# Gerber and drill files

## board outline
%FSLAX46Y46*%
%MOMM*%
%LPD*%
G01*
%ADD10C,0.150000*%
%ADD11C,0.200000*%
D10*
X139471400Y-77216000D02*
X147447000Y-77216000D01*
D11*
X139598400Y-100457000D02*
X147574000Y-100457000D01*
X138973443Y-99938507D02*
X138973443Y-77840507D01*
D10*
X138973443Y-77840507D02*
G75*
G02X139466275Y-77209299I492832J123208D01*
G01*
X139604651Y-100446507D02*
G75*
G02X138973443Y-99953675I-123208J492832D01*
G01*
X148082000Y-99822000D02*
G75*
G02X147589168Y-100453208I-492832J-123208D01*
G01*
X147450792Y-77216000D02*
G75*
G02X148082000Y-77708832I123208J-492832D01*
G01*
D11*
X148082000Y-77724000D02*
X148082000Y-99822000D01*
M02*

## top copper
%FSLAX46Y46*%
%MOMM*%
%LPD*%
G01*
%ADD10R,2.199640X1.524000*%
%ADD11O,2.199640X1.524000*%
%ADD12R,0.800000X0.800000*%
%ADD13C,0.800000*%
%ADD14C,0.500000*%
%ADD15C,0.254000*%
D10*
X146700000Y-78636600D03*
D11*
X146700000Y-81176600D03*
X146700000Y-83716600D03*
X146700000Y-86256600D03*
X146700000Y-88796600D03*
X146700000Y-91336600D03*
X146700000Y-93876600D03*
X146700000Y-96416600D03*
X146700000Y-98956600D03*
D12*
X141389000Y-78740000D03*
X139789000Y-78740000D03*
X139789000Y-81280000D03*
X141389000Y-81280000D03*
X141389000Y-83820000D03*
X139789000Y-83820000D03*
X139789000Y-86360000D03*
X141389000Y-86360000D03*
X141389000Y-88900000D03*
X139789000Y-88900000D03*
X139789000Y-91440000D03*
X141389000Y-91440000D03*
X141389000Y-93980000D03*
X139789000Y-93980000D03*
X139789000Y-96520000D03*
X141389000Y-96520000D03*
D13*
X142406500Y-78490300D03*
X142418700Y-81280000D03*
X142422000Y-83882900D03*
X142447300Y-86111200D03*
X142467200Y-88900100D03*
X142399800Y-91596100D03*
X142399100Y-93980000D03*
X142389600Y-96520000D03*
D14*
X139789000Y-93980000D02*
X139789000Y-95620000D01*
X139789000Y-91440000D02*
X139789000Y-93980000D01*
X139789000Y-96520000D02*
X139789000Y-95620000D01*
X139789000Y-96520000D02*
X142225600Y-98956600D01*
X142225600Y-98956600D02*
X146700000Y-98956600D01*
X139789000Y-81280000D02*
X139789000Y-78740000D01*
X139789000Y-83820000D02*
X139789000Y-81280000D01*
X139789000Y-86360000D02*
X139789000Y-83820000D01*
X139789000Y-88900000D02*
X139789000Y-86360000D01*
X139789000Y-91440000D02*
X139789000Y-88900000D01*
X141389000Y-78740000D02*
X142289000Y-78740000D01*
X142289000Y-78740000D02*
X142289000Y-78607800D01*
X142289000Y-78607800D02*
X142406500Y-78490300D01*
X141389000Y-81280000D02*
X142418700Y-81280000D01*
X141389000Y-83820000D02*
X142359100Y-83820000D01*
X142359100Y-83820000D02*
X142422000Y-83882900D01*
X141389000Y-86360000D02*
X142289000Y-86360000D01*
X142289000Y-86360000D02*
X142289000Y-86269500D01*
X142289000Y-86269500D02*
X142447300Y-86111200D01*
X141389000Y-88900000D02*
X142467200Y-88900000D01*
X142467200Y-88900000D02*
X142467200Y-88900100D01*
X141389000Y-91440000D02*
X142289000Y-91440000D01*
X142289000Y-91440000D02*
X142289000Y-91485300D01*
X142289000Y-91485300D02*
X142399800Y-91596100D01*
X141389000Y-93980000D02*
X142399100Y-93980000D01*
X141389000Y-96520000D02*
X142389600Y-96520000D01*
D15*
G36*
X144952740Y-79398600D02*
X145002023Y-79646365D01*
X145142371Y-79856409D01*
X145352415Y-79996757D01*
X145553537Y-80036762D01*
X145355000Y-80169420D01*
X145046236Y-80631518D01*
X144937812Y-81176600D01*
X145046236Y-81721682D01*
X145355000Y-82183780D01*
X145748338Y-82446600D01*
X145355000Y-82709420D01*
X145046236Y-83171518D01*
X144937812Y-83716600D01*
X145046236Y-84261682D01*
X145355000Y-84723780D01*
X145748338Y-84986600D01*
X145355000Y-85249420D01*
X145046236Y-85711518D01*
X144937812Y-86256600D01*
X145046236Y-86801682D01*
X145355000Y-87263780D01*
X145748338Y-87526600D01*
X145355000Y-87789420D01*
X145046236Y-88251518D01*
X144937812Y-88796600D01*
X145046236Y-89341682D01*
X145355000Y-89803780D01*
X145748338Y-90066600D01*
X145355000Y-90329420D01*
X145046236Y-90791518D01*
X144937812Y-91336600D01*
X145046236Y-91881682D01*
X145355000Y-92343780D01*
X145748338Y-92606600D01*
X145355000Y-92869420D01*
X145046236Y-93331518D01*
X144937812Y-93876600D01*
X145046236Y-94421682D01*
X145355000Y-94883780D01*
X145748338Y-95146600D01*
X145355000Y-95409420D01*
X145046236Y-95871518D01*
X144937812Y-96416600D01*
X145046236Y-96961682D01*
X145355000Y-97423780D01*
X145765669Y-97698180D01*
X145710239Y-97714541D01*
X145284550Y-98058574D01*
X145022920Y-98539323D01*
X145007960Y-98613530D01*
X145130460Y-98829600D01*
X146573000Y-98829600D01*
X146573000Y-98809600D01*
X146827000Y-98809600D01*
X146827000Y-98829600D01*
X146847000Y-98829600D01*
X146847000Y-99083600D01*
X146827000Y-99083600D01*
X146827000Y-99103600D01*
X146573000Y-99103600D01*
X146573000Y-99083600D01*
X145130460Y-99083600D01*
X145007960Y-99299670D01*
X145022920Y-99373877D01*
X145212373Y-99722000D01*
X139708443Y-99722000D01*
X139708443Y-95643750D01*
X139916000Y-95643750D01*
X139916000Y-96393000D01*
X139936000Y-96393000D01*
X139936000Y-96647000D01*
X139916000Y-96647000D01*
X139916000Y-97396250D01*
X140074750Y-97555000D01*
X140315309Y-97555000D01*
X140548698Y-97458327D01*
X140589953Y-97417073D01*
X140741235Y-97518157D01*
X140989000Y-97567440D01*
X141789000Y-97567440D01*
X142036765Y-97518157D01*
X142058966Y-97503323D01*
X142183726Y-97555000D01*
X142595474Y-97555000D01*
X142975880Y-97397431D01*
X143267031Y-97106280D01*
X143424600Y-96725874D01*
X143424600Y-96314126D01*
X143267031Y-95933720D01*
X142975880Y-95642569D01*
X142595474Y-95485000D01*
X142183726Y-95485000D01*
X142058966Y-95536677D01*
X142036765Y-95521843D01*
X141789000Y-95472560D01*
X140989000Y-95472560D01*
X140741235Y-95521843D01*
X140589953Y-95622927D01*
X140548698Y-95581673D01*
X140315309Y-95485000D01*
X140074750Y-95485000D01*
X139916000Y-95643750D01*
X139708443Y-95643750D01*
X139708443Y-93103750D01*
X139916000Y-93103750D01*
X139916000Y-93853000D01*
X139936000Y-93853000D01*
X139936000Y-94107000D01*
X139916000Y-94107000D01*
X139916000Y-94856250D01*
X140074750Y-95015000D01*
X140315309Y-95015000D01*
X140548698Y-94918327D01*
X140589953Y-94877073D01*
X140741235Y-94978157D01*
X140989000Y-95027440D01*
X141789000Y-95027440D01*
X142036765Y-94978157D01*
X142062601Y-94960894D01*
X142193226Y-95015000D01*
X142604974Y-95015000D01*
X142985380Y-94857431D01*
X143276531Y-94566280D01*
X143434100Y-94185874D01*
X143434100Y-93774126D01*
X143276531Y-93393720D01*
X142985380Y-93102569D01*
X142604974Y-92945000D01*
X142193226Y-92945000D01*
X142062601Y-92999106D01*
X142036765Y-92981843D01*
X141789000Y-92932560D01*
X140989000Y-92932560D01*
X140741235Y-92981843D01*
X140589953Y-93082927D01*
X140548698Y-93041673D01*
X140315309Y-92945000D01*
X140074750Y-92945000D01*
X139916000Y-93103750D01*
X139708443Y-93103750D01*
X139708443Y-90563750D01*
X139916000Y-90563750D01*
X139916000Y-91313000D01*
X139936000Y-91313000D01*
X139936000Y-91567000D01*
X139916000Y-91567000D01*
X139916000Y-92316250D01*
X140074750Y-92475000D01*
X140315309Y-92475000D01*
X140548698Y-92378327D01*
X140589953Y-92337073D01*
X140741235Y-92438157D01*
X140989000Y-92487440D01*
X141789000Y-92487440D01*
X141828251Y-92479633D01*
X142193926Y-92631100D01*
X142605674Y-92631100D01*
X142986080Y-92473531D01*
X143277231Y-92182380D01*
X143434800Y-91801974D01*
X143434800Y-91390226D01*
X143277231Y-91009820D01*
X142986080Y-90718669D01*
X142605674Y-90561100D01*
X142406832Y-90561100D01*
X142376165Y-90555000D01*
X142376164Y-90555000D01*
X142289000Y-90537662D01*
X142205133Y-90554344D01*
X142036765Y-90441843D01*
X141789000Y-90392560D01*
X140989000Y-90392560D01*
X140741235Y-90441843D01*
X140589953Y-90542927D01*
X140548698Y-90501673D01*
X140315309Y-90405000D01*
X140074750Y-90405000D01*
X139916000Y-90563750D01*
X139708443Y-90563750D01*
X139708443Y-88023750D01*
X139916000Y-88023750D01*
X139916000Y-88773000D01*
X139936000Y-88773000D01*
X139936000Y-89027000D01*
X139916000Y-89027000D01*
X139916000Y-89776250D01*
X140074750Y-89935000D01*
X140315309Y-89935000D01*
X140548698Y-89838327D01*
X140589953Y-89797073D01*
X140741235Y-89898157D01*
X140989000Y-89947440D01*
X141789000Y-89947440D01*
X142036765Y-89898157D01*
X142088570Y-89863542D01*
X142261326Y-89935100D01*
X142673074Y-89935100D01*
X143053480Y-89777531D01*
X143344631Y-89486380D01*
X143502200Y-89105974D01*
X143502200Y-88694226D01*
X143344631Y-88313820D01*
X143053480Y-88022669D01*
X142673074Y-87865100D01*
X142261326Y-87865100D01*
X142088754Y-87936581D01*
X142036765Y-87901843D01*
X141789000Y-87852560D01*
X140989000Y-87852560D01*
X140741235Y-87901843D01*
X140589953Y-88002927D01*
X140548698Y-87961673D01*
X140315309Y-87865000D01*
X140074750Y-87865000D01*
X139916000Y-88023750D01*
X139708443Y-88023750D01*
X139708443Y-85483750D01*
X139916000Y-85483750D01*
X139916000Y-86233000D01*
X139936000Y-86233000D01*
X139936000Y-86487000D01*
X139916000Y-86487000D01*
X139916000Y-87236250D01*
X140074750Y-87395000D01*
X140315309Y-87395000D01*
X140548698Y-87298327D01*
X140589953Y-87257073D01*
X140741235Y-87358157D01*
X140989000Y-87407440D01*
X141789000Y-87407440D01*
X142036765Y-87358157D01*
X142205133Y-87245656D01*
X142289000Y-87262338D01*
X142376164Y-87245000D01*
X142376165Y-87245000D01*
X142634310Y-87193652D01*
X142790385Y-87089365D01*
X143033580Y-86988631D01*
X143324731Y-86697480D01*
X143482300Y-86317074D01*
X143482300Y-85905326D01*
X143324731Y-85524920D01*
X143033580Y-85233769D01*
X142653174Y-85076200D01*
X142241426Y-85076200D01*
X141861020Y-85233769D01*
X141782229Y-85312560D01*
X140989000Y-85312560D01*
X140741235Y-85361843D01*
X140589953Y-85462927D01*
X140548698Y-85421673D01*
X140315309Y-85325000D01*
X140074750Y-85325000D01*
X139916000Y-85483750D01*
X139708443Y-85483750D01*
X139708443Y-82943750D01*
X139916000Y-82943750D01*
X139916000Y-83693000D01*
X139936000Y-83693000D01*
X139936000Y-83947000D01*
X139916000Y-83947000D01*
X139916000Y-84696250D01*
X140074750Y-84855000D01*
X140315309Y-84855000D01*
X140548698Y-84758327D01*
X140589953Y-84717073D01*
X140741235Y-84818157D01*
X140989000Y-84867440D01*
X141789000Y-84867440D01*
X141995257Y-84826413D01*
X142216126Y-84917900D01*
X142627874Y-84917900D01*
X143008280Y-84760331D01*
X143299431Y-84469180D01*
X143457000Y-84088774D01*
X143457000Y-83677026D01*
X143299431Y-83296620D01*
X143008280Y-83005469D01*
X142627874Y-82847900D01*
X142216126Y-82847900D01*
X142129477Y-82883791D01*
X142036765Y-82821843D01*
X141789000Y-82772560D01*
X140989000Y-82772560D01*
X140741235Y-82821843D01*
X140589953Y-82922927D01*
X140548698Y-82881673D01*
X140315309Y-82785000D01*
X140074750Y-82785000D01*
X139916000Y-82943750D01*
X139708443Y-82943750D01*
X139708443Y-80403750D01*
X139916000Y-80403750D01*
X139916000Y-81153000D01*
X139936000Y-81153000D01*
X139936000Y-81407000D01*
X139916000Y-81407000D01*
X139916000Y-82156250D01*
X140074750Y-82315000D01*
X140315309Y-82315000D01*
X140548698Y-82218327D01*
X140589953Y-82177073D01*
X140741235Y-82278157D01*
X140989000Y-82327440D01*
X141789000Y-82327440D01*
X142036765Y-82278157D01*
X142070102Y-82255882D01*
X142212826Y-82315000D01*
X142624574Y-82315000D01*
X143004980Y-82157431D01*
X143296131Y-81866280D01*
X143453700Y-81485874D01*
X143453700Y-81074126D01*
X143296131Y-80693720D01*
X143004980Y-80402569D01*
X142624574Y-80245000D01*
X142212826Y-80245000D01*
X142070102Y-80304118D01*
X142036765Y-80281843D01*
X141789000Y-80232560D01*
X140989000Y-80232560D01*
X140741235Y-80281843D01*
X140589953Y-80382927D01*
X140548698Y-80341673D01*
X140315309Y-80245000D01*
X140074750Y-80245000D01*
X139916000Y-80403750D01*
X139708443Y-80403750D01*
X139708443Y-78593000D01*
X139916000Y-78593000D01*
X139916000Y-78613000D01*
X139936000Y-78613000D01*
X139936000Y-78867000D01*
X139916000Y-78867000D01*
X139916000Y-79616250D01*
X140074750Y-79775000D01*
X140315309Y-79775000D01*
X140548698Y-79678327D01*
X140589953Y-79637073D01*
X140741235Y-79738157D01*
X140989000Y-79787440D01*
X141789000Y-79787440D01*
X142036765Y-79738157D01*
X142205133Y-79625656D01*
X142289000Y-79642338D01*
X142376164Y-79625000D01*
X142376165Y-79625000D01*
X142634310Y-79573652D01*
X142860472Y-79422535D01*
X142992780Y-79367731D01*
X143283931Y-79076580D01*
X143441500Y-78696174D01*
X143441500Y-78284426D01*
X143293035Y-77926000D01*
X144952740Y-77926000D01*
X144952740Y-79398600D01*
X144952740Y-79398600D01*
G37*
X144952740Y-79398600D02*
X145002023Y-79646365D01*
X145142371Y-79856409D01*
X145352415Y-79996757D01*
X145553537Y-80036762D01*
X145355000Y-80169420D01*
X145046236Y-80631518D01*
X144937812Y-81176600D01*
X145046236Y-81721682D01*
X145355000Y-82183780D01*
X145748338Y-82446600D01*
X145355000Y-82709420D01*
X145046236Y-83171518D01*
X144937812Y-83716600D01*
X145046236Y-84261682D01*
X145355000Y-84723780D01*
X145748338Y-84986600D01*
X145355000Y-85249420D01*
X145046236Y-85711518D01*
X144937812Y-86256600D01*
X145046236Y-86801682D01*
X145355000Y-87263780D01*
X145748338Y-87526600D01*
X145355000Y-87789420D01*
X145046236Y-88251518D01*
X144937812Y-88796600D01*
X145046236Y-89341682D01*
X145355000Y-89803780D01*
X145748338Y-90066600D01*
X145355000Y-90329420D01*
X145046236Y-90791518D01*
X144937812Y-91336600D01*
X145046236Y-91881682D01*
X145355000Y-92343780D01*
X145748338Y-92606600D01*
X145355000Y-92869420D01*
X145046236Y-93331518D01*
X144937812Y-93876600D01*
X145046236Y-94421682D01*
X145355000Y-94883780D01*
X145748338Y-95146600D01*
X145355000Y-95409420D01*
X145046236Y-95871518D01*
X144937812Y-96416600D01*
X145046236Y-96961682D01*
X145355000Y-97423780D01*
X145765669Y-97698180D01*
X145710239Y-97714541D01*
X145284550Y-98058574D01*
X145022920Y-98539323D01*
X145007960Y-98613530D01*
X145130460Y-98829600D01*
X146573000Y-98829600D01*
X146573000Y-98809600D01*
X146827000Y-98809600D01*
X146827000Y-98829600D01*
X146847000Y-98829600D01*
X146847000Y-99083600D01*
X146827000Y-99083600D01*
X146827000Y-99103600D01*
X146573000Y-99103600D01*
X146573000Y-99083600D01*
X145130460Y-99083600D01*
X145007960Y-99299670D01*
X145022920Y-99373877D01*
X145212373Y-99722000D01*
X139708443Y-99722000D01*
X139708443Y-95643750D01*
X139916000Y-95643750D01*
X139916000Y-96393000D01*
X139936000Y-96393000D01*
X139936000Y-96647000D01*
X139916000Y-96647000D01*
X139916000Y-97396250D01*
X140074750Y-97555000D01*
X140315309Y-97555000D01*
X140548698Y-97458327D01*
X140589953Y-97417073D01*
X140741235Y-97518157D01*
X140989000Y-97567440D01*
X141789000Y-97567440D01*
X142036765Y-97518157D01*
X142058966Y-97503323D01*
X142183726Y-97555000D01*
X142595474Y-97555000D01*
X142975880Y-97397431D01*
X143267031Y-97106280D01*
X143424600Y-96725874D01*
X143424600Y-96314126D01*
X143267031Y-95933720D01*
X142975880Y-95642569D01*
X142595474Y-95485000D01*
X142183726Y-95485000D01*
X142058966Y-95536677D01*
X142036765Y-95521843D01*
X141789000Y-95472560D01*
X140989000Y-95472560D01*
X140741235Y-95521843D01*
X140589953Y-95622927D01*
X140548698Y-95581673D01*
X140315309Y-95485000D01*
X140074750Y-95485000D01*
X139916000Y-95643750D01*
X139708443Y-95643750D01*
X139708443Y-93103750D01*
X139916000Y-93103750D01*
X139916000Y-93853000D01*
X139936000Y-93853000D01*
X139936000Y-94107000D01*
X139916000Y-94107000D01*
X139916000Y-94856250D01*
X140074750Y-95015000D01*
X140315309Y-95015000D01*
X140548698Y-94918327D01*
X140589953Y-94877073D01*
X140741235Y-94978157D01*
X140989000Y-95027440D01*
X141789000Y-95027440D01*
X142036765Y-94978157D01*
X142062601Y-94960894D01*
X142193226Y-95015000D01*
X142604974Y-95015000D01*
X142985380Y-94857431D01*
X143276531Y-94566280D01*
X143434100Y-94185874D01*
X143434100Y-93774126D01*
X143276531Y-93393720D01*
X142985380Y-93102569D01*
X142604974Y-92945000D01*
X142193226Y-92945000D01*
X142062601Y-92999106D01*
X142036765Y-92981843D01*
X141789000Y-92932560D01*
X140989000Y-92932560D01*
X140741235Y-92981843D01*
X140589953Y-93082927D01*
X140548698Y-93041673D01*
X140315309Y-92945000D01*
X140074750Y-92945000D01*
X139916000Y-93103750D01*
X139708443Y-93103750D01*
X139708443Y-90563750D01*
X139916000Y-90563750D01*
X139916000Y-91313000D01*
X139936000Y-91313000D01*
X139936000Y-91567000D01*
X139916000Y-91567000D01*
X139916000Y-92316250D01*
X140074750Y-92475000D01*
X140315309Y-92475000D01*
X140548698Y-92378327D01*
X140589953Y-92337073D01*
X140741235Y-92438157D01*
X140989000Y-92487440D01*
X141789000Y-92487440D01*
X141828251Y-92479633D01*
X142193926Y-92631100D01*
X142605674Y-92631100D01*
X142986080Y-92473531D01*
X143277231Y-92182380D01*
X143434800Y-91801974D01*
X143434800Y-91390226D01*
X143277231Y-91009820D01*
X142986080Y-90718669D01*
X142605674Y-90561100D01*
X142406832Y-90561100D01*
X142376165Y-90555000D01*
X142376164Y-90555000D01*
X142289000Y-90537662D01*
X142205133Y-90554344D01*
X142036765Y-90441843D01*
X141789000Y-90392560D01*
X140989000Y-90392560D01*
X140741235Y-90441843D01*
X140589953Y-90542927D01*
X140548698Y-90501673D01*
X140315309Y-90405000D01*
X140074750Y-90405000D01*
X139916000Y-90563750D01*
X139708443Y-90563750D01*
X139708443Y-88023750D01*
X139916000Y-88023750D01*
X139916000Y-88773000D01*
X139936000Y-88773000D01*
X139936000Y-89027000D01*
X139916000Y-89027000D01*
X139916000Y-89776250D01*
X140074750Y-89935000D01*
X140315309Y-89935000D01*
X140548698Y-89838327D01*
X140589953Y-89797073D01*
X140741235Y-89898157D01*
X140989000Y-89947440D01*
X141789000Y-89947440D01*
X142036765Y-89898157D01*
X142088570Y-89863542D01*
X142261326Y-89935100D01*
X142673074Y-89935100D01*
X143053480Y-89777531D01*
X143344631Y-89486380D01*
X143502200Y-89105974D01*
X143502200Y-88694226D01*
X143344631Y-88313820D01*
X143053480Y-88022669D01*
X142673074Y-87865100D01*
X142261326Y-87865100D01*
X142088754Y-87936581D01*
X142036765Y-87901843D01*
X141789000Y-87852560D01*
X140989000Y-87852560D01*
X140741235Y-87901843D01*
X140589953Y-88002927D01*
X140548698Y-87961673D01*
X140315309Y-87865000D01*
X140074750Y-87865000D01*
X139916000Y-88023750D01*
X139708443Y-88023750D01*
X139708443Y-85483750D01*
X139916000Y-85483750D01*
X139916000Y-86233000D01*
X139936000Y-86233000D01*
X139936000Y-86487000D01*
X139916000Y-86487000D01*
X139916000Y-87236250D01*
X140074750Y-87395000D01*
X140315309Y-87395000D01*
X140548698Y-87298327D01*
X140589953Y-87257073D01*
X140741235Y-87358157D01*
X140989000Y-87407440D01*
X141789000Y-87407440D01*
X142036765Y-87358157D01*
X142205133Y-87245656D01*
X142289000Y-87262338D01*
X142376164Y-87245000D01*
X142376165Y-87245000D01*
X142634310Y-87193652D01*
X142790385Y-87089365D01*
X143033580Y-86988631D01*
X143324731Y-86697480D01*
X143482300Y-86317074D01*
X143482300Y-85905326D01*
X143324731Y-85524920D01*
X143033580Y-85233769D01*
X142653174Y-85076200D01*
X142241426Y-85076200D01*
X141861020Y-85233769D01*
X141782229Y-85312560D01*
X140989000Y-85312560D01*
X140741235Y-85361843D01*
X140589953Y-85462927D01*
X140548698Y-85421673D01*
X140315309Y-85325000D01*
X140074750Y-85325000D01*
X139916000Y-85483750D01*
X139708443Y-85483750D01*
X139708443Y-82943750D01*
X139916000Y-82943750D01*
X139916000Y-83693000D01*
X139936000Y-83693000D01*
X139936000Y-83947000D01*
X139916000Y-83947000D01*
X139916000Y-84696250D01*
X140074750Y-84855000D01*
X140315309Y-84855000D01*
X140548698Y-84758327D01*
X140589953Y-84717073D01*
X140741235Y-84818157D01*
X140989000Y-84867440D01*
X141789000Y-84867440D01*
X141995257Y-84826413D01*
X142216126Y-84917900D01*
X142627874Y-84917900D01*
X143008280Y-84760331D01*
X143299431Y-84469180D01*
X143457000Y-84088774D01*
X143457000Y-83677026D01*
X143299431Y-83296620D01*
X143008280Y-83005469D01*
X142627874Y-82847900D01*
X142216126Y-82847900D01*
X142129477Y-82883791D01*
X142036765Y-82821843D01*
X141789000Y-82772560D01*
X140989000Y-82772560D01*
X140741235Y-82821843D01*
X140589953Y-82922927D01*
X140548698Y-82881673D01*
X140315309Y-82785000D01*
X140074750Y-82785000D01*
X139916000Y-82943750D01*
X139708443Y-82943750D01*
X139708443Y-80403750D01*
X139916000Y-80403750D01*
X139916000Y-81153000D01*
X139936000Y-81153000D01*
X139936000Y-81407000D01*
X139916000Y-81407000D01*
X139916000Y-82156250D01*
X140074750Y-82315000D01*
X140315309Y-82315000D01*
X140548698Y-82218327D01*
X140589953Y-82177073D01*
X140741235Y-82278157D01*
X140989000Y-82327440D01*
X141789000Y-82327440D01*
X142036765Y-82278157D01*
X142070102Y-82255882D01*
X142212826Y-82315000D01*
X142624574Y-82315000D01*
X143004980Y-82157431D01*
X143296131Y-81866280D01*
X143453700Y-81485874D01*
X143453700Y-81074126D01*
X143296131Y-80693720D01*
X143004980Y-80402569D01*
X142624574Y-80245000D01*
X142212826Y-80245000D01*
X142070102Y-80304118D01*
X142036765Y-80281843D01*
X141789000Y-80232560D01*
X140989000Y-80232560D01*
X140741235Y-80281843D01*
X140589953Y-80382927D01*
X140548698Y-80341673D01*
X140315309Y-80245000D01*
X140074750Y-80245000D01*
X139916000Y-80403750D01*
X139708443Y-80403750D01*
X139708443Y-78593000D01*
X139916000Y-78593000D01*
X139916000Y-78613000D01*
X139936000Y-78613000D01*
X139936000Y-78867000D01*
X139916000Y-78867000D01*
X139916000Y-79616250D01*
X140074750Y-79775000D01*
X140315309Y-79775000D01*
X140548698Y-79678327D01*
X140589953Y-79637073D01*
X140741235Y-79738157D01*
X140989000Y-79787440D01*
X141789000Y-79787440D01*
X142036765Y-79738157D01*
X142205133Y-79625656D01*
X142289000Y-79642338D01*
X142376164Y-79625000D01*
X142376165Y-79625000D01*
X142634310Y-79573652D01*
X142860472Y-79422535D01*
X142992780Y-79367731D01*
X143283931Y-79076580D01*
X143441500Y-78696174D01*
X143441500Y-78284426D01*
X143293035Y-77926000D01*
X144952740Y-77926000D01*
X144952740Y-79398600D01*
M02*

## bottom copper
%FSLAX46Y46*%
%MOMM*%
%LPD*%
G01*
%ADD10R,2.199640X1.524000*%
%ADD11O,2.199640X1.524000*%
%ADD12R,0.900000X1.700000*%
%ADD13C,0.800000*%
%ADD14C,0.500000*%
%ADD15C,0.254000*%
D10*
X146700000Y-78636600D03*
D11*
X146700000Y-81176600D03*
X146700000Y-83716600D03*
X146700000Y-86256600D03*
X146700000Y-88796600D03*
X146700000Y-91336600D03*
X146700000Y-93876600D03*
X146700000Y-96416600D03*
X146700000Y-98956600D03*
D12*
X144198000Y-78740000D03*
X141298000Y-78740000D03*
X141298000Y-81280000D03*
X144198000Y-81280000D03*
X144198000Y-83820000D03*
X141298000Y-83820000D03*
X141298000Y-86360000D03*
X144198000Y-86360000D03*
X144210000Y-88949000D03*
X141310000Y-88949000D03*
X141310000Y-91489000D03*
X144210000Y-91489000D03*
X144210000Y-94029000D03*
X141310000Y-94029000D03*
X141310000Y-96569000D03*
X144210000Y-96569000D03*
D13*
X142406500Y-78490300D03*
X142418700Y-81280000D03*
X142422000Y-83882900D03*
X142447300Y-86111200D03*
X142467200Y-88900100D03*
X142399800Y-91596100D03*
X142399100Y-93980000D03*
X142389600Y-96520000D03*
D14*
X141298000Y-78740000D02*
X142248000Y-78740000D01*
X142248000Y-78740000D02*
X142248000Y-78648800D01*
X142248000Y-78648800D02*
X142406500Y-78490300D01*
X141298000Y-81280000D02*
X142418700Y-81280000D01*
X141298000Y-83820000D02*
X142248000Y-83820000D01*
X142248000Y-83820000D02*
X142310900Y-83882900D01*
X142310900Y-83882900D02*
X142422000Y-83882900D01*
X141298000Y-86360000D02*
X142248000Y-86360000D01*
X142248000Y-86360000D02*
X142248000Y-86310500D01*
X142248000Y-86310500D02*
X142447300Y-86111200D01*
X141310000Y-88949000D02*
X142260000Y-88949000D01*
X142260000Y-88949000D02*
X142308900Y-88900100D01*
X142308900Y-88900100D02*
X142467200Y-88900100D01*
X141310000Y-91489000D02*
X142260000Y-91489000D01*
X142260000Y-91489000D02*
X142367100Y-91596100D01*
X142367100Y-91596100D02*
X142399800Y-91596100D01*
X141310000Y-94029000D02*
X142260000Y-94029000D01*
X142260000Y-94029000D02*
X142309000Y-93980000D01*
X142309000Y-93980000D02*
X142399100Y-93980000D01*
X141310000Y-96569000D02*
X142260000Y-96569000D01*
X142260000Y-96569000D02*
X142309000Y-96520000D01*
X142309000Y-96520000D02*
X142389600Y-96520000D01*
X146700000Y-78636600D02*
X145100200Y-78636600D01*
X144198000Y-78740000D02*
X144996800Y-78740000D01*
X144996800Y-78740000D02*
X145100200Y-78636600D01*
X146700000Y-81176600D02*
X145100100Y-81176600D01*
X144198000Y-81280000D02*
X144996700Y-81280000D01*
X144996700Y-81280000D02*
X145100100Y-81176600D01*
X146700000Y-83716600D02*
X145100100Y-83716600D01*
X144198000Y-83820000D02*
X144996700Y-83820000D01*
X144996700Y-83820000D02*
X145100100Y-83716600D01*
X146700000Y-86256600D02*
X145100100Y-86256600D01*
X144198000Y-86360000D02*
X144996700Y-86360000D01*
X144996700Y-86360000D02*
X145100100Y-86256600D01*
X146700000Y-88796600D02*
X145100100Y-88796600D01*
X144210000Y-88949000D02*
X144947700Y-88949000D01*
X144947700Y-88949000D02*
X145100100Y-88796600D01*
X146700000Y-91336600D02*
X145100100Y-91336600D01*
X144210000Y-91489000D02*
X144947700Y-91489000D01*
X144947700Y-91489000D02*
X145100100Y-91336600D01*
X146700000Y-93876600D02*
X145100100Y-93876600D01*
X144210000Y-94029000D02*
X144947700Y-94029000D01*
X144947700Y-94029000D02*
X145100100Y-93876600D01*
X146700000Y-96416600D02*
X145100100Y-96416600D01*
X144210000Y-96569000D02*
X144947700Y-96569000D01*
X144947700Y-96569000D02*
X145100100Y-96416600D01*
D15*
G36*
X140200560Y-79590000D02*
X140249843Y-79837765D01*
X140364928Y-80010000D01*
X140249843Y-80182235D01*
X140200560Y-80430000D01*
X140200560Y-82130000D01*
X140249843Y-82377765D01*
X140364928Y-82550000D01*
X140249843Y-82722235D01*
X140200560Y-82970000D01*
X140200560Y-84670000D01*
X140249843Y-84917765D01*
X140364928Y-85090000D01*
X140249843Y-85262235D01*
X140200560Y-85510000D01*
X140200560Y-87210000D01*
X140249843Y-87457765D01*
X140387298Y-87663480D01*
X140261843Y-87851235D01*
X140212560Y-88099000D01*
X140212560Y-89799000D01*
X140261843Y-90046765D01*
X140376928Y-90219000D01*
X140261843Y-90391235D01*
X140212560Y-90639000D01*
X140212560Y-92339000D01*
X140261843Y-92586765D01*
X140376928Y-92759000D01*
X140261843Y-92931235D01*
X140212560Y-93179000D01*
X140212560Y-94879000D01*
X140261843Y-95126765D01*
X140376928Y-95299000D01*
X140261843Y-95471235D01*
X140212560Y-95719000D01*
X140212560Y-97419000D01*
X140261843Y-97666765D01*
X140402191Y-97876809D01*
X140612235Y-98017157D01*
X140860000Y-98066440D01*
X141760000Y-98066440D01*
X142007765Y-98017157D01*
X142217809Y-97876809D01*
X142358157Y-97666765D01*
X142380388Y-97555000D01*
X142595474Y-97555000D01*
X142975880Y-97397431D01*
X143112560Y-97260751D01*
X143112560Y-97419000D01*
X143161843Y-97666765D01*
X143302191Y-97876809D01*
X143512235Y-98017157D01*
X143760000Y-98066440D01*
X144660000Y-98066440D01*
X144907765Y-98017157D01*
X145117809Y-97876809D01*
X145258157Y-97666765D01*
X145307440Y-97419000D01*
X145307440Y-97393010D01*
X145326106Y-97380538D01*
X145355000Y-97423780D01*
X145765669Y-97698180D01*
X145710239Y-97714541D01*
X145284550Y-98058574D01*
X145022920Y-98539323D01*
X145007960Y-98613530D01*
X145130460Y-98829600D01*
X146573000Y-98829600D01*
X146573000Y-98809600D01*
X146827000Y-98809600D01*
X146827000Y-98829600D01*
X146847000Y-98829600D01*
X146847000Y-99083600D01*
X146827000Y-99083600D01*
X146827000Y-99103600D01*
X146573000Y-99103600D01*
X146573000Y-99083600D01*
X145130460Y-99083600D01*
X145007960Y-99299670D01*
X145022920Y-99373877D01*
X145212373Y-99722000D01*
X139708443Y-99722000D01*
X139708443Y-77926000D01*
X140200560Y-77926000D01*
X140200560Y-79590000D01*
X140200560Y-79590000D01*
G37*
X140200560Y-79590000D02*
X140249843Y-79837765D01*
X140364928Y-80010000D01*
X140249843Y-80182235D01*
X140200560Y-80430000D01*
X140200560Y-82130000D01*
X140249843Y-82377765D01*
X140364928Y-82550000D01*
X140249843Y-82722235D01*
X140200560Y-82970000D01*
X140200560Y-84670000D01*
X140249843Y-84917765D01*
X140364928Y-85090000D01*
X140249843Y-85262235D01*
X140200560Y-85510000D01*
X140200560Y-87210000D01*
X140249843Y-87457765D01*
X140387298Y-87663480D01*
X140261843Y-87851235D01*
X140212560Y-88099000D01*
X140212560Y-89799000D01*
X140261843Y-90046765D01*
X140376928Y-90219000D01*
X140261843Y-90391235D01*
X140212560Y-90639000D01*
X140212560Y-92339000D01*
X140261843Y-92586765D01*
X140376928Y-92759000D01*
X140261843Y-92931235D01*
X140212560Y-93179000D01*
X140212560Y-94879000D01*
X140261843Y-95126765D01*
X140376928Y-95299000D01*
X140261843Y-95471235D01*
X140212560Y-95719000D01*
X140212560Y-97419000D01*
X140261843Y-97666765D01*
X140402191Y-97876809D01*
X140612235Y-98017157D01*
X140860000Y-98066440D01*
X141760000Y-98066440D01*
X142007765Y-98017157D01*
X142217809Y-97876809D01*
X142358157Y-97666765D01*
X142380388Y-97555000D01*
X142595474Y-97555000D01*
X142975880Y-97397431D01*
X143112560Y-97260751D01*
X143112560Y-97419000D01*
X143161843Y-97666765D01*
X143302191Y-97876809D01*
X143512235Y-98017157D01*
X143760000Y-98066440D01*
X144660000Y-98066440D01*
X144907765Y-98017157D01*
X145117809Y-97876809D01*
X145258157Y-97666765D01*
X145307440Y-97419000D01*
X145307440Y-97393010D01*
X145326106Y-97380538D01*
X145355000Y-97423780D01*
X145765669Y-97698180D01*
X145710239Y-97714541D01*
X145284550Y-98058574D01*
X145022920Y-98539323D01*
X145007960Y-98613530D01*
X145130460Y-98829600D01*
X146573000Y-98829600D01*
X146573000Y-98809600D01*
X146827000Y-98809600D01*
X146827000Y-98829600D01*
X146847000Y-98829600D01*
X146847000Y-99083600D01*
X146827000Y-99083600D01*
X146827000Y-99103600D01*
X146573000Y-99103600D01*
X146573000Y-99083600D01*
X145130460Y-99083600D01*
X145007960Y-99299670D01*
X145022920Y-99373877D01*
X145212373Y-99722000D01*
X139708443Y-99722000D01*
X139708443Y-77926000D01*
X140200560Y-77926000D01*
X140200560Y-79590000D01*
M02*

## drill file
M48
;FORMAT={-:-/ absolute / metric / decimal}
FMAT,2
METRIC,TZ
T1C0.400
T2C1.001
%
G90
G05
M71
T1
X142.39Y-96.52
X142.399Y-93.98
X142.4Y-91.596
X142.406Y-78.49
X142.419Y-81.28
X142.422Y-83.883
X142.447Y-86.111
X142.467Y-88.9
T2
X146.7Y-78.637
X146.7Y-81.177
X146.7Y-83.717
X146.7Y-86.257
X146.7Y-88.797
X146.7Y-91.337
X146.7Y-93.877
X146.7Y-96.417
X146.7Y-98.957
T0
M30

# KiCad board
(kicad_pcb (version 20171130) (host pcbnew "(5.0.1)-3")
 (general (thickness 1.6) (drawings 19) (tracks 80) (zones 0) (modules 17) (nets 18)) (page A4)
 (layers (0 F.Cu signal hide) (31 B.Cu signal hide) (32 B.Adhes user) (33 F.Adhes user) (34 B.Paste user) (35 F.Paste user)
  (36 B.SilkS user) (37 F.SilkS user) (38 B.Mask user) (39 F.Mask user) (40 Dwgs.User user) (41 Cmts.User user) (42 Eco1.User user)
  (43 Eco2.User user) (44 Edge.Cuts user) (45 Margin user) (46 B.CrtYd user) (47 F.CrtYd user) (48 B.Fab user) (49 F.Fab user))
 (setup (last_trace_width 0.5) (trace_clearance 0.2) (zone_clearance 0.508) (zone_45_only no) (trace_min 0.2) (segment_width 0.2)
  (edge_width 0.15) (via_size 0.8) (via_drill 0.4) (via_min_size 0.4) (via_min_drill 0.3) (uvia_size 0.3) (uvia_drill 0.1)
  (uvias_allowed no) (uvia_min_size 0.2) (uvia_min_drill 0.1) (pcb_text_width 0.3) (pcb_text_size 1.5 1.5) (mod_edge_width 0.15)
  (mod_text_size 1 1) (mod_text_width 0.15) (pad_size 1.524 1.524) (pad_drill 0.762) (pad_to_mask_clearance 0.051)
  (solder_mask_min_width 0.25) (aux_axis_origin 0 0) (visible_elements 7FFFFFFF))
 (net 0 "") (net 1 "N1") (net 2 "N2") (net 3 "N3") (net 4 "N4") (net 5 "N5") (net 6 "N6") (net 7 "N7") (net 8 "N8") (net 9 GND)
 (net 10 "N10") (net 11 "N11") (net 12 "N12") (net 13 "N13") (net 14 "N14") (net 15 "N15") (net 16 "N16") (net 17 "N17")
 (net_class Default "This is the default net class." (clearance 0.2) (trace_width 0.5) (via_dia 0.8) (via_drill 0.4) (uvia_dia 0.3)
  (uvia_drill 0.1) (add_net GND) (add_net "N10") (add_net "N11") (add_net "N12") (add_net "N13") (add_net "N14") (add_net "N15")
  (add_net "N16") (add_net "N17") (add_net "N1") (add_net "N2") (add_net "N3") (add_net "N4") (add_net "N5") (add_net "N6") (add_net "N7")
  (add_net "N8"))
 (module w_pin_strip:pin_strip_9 (layer B.Cu) (at 146.7 88.7966 270)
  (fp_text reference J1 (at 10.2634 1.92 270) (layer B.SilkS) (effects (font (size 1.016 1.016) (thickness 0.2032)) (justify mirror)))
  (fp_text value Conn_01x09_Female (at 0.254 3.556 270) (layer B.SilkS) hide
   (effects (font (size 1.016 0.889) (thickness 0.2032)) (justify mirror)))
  (pad 1 thru_hole rect (at -10.16 0 270) (size 1.524 2.19964) (drill 1.00076) (layers *.Cu *.Mask B.SilkS) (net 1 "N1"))
  (pad 2 thru_hole oval (at -7.62 0 270) (size 1.524 2.19964) (drill 1.00076) (layers *.Cu *.Mask B.SilkS) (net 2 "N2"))
  (pad 3 thru_hole oval (at -5.08 0 270) (size 1.524 2.19964) (drill 1.00076) (layers *.Cu *.Mask B.SilkS) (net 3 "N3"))
  (pad 4 thru_hole oval (at -2.54 0 270) (size 1.524 2.19964) (drill 1.00076) (layers *.Cu *.Mask B.SilkS) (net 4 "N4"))
  (pad 5 thru_hole oval (at 0 0 270) (size 1.524 2.19964) (drill 1.00076) (layers *.Cu *.Mask B.SilkS) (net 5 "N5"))
  (pad 6 thru_hole oval (at 2.54 0 270) (size 1.524 2.19964) (drill 1.00076) (layers *.Cu *.Mask B.SilkS) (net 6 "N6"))
  (pad 7 thru_hole oval (at 5.08 0 270) (size 1.524 2.19964) (drill 1.00076) (layers *.Cu *.Mask B.SilkS) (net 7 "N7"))
  (pad 8 thru_hole oval (at 7.62 0 270) (size 1.524 2.19964) (drill 1.00076) (layers *.Cu *.Mask B.SilkS) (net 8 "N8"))
  (pad 9 thru_hole oval (at 10.16 0 270) (size 1.524 2.19964) (drill 1.00076) (layers *.Cu *.Mask B.SilkS) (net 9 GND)))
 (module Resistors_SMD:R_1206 (layer B.Cu) (at 142.748 78.74 180)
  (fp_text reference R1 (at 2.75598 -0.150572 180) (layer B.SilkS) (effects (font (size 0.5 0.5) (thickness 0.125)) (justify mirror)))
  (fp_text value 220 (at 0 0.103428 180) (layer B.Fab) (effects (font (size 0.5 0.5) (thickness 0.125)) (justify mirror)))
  (pad 1 smd rect (at -1.45 0 180) (size 0.9 1.7) (layers B.Cu B.Paste B.Mask) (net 1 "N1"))
  (pad 2 smd rect (at 1.45 0 180) (size 0.9 1.7) (layers B.Cu B.Paste B.Mask) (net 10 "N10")))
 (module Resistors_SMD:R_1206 (layer B.Cu) (at 142.748 81.28 180)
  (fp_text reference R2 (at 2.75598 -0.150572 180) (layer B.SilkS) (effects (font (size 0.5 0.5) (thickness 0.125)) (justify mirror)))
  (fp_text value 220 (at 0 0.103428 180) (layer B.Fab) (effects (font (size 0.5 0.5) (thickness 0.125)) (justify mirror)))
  (pad 2 smd rect (at 1.45 0 180) (size 0.9 1.7) (layers B.Cu B.Paste B.Mask) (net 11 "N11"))
  (pad 1 smd rect (at -1.45 0 180) (size 0.9 1.7) (layers B.Cu B.Paste B.Mask) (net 2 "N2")))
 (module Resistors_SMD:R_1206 (layer B.Cu) (at 142.748 83.82 180)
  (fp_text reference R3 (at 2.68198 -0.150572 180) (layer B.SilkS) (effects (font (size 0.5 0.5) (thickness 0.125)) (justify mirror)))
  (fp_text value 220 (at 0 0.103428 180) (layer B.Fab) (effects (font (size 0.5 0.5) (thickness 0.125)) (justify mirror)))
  (pad 1 smd rect (at -1.45 0 180) (size 0.9 1.7) (layers B.Cu B.Paste B.Mask) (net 3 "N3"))
  (pad 2 smd rect (at 1.45 0 180) (size 0.9 1.7) (layers B.Cu B.Paste B.Mask) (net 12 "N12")))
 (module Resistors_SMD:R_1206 (layer B.Cu) (at 142.748 86.36 180)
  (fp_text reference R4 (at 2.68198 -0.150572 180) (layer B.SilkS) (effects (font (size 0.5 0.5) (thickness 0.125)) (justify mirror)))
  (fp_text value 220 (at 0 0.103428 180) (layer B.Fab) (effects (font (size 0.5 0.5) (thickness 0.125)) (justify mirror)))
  (pad 2 smd rect (at 1.45 0 180) (size 0.9 1.7) (layers B.Cu B.Paste B.Mask) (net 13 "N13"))
  (pad 1 smd rect (at -1.45 0 180) (size 0.9 1.7) (layers B.Cu B.Paste B.Mask) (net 4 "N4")))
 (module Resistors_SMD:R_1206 (layer B.Cu) (at 142.76 88.949 180)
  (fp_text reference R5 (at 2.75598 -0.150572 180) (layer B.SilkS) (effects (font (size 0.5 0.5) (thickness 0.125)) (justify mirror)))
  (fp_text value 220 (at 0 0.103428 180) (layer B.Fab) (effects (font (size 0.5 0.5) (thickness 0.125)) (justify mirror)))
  (pad 1 smd rect (at -1.45 0 180) (size 0.9 1.7) (layers B.Cu B.Paste B.Mask) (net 5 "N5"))
  (pad 2 smd rect (at 1.45 0 180) (size 0.9 1.7) (layers B.Cu B.Paste B.Mask) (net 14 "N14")))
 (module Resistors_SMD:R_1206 (layer B.Cu) (at 142.76 91.489 180)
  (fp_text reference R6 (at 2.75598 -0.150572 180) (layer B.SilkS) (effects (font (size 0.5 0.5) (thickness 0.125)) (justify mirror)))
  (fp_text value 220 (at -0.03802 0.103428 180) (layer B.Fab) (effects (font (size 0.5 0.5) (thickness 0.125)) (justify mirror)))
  (pad 2 smd rect (at 1.45 0 180) (size 0.9 1.7) (layers B.Cu B.Paste B.Mask) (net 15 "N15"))
  (pad 1 smd rect (at -1.45 0 180) (size 0.9 1.7) (layers B.Cu B.Paste B.Mask) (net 6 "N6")))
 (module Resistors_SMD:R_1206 (layer B.Cu) (at 142.76 94.029 180)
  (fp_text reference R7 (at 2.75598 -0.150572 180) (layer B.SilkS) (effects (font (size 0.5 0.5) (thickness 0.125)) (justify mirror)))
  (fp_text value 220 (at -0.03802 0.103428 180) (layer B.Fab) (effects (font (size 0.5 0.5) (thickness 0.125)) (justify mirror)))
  (pad 1 smd rect (at -1.45 0 180) (size 0.9 1.7) (layers B.Cu B.Paste B.Mask) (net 7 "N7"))
  (pad 2 smd rect (at 1.45 0 180) (size 0.9 1.7) (layers B.Cu B.Paste B.Mask) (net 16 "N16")))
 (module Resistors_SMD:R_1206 (layer B.Cu) (at 142.76 96.569 180)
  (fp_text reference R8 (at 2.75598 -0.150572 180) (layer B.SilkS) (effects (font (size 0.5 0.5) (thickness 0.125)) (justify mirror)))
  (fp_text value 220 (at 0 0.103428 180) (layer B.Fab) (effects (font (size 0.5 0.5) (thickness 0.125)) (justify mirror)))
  (pad 2 smd rect (at 1.45 0 180) (size 0.9 1.7) (layers B.Cu B.Paste B.Mask) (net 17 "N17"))
  (pad 1 smd rect (at -1.45 0 180) (size 0.9 1.7) (layers B.Cu B.Paste B.Mask) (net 8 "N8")))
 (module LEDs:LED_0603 (layer F.Cu) (at 140.589 78.74)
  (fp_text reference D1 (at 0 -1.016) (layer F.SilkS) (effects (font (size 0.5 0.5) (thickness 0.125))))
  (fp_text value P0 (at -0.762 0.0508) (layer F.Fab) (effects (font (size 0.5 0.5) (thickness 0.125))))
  (pad 2 smd rect (at 0.8 0 180) (size 0.8 0.8) (layers F.Cu F.Paste F.Mask) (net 10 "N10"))
  (pad 1 smd rect (at -0.8 0 180) (size 0.8 0.8) (layers F.Cu F.Paste F.Mask) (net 9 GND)))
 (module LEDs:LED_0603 (layer F.Cu) (at 140.589 81.28)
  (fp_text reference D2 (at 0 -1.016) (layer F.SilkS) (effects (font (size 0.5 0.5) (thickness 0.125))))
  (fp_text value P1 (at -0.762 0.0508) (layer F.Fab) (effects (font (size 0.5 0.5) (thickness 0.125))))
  (pad 1 smd rect (at -0.8 0 180) (size 0.8 0.8) (layers F.Cu F.Paste F.Mask) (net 9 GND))
  (pad 2 smd rect (at 0.8 0 180) (size 0.8 0.8) (layers F.Cu F.Paste F.Mask) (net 11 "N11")))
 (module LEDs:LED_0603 (layer F.Cu) (at 140.589 83.82)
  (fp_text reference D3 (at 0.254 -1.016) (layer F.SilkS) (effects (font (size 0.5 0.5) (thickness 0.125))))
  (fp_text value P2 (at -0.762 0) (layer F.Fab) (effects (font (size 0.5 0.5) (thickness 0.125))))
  (pad 2 smd rect (at 0.8 0 180) (size 0.8 0.8) (layers F.Cu F.Paste F.Mask) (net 12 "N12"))
  (pad 1 smd rect (at -0.8 0 180) (size 0.8 0.8) (layers F.Cu F.Paste F.Mask) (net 9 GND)))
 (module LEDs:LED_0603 (layer F.Cu) (at 140.589 86.36)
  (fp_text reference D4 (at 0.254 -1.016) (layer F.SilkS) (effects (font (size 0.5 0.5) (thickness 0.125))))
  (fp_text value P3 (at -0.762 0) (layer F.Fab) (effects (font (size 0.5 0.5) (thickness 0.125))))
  (pad 1 smd rect (at -0.8 0 180) (size 0.8 0.8) (layers F.Cu F.Paste F.Mask) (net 9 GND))
  (pad 2 smd rect (at 0.8 0 180) (size 0.8 0.8) (layers F.Cu F.Paste F.Mask) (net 13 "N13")))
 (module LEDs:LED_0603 (layer F.Cu) (at 140.589 88.9)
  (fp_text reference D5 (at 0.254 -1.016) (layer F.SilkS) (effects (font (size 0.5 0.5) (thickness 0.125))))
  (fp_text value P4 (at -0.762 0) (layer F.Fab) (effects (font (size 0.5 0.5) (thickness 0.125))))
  (pad 2 smd rect (at 0.8 0 180) (size 0.8 0.8) (layers F.Cu F.Paste F.Mask) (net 14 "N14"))
  (pad 1 smd rect (at -0.8 0 180) (size 0.8 0.8) (layers F.Cu F.Paste F.Mask) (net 9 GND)))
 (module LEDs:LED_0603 (layer F.Cu) (at 140.589 91.44)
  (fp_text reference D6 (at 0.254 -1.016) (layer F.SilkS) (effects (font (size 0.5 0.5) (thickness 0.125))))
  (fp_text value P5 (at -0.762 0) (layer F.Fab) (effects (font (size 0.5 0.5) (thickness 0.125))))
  (pad 1 smd rect (at -0.8 0 180) (size 0.8 0.8) (layers F.Cu F.Paste F.Mask) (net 9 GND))
  (pad 2 smd rect (at 0.8 0 180) (size 0.8 0.8) (layers F.Cu F.Paste F.Mask) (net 15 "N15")))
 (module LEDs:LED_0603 (layer F.Cu) (at 140.589 93.98)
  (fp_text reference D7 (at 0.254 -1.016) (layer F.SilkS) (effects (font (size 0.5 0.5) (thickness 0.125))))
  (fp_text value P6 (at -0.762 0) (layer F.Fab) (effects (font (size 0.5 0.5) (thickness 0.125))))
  (pad 2 smd rect (at 0.8 0 180) (size 0.8 0.8) (layers F.Cu F.Paste F.Mask) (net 16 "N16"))
  (pad 1 smd rect (at -0.8 0 180) (size 0.8 0.8) (layers F.Cu F.Paste F.Mask) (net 9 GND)))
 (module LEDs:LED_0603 (layer F.Cu) (at 140.589 96.52)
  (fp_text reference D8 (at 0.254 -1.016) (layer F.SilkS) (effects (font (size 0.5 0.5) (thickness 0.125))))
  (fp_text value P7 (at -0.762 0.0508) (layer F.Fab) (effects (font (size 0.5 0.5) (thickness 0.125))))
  (pad 1 smd rect (at -0.8 0 180) (size 0.8 0.8) (layers F.Cu F.Paste F.Mask) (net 9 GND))
  (pad 2 smd rect (at 0.8 0 180) (size 0.8 0.8) (layers F.Cu F.Paste F.Mask) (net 17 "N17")))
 (gr_line (start 139.4714 77.216) (end 147.447 77.216) (layer Edge.Cuts) (width 0.15))
 (gr_line (start 139.5984 100.457) (end 147.574 100.457) (layer Edge.Cuts) (width 0.2))
 (gr_line (start 138.973443 99.938507) (end 138.973443 77.840507) (layer Edge.Cuts) (width 0.2))
 (gr_arc (start 139.466275 77.717299) (end 139.466275 77.209299) (angle -104.0362435) (layer Edge.Cuts) (width 0.15))
 (gr_arc (start 139.481443 99.953675) (end 138.973443 99.953675) (angle -104.0362435) (layer Edge.Cuts) (width 0.15))
 (gr_arc (start 147.589168 99.945208) (end 147.589168 100.453208) (angle -104.0362435) (layer Edge.Cuts) (width 0.15))
 (gr_arc (start 147.574 77.708832) (end 148.082 77.708832) (angle -104.0362435) (layer Edge.Cuts) (width 0.15))
 (gr_line (start 148.082 77.724) (end 148.082 99.822) (layer Edge.Cuts) (width 0.2))
 (segment (start 139.789 93.98) (end 139.789 95.62) (width 0.5) (layer F.Cu) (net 9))
 (segment (start 139.789 91.44) (end 139.789 93.98) (width 0.5) (layer F.Cu) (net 9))
 (segment (start 139.789 96.52) (end 139.789 95.62) (width 0.5) (layer F.Cu) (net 9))
 (segment (start 139.789 96.52) (end 142.2256 98.9566) (width 0.5) (layer F.Cu) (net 9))
 (segment (start 142.2256 98.9566) (end 146.7 98.9566) (width 0.5) (layer F.Cu) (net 9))
 (segment (start 139.789 81.28) (end 139.789 78.74) (width 0.5) (layer F.Cu) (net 9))
 (segment (start 139.789 83.82) (end 139.789 81.28) (width 0.5) (layer F.Cu) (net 9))
 (segment (start 139.789 86.36) (end 139.789 83.82) (width 0.5) (layer F.Cu) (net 9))
 (segment (start 139.789 88.9) (end 139.789 86.36) (width 0.5) (layer F.Cu) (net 9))
 (segment (start 139.789 91.44) (end 139.789 88.9) (width 0.5) (layer F.Cu) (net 9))
 (segment (start 141.298 78.74) (end 142.248 78.74) (width 0.5) (layer B.Cu) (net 10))
 (segment (start 141.389 78.74) (end 142.289 78.74) (width 0.5) (layer F.Cu) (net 10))
 (segment (start 142.289 78.74) (end 142.289 78.6078) (width 0.5) (layer F.Cu) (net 10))
 (segment (start 142.289 78.6078) (end 142.4065 78.4903) (width 0.5) (layer F.Cu) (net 10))
 (segment (start 142.248 78.74) (end 142.248 78.6488) (width 0.5) (layer B.Cu) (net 10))
 (segment (start 142.248 78.6488) (end 142.4065 78.4903) (width 0.5) (layer B.Cu) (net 10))
 (via (at 142.4065 78.4903) (size 0.8) (layers F.Cu B.Cu) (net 10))
 (segment (start 141.389 81.28) (end 142.4187 81.28) (width 0.5) (layer F.Cu) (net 11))
 (segment (start 141.298 81.28) (end 142.4187 81.28) (width 0.5) (layer B.Cu) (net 11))
 (via (at 142.4187 81.28) (size 0.8) (layers F.Cu B.Cu) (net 11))
 (segment (start 141.298 83.82) (end 142.248 83.82) (width 0.5) (layer B.Cu) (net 12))
 (segment (start 141.389 83.82) (end 142.3591 83.82) (width 0.5) (layer F.Cu) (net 12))
 (segment (start 142.3591 83.82) (end 142.422 83.8829) (width 0.5) (layer F.Cu) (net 12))
 (segment (start 142.248 83.82) (end 142.3109 83.8829) (width 0.5) (layer B.Cu) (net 12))
 (segment (start 142.3109 83.8829) (end 142.422 83.8829) (width 0.5) (layer B.Cu) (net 12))
 (via (at 142.422 83.8829) (size 0.8) (layers F.Cu B.Cu) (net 12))
 (segment (start 141.298 86.36) (end 142.248 86.36) (width 0.5) (layer B.Cu) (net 13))
 (segment (start 141.389 86.36) (end 142.289 86.36) (width 0.5) (layer F.Cu) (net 13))
 (segment (start 142.289 86.36) (end 142.289 86.2695) (width 0.5) (layer F.Cu) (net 13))
 (segment (start 142.289 86.2695) (end 142.4473 86.1112) (width 0.5) (layer F.Cu) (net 13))
 (segment (start 142.248 86.36) (end 142.248 86.3105) (width 0.5) (layer B.Cu) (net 13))
 (segment (start 142.248 86.3105) (end 142.4473 86.1112) (width 0.5) (layer B.Cu) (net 13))
 (via (at 142.4473 86.1112) (size 0.8) (layers F.Cu B.Cu) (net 13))
 (segment (start 141.31 88.949) (end 142.26 88.949) (width 0.5) (layer B.Cu) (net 14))
 (segment (start 141.389 88.9) (end 142.4672 88.9) (width 0.5) (layer F.Cu) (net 14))
 (segment (start 142.4672 88.9) (end 142.4672 88.9001) (width 0.5) (layer F.Cu) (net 14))
 (segment (start 142.26 88.949) (end 142.3089 88.9001) (width 0.5) (layer B.Cu) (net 14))
 (segment (start 142.3089 88.9001) (end 142.4672 88.9001) (width 0.5) (layer B.Cu) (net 14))
 (via (at 142.4672 88.9001) (size 0.8) (layers F.Cu B.Cu) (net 14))
 (segment (start 141.31 91.489) (end 142.26 91.489) (width 0.5) (layer B.Cu) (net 15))
 (segment (start 141.389 91.44) (end 142.289 91.44) (width 0.5) (layer F.Cu) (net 15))
 (segment (start 142.289 91.44) (end 142.289 91.4853) (width 0.5) (layer F.Cu) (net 15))
 (segment (start 142.289 91.4853) (end 142.3998 91.5961) (width 0.5) (layer F.Cu) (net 15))
 (segment (start 142.26 91.489) (end 142.3671 91.5961) (width 0.5) (layer B.Cu) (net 15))
 (segment (start 142.3671 91.5961) (end 142.3998 91.5961) (width 0.5) (layer B.Cu) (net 15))
 (via (at 142.3998 91.5961) (size 0.8) (layers F.Cu B.Cu) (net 15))
 (segment (start 141.31 94.029) (end 142.26 94.029) (width 0.5) (layer B.Cu) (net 16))
 (segment (start 141.389 93.98) (end 142.3991 93.98) (width 0.5) (layer F.Cu) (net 16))
 (segment (start 142.26 94.029) (end 142.309 93.98) (width 0.5) (layer B.Cu) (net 16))
 (segment (start 142.309 93.98) (end 142.3991 93.98) (width 0.5) (layer B.Cu) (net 16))
 (via (at 142.3991 93.98) (size 0.8) (layers F.Cu B.Cu) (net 16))
 (segment (start 141.31 96.569) (end 142.26 96.569) (width 0.5) (layer B.Cu) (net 17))
 (segment (start 141.389 96.52) (end 142.3896 96.52) (width 0.5) (layer F.Cu) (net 17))
 (segment (start 142.26 96.569) (end 142.309 96.52) (width 0.5) (layer B.Cu) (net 17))
 (segment (start 142.309 96.52) (end 142.3896 96.52) (width 0.5) (layer B.Cu) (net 17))
 (via (at 142.3896 96.52) (size 0.8) (layers F.Cu B.Cu) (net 17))
 (segment (start 146.7 78.6366) (end 145.1002 78.6366) (width 0.5) (layer B.Cu) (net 1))
 (segment (start 144.198 78.74) (end 144.9968 78.74) (width 0.5) (layer B.Cu) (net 1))
 (segment (start 144.9968 78.74) (end 145.1002 78.6366) (width 0.5) (layer B.Cu) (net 1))
 (segment (start 146.7 81.1766) (end 145.1001 81.1766) (width 0.5) (layer B.Cu) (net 2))
 (segment (start 144.198 81.28) (end 144.9967 81.28) (width 0.5) (layer B.Cu) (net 2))
 (segment (start 144.9967 81.28) (end 145.1001 81.1766) (width 0.5) (layer B.Cu) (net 2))
 (segment (start 146.7 83.7166) (end 145.1001 83.7166) (width 0.5) (layer B.Cu) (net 3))
 (segment (start 144.198 83.82) (end 144.9967 83.82) (width 0.5) (layer B.Cu) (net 3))
 (segment (start 144.9967 83.82) (end 145.1001 83.7166) (width 0.5) (layer B.Cu) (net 3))
 (segment (start 146.7 86.2566) (end 145.1001 86.2566) (width 0.5) (layer B.Cu) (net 4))
 (segment (start 144.198 86.36) (end 144.9967 86.36) (width 0.5) (layer B.Cu) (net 4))
 (segment (start 144.9967 86.36) (end 145.1001 86.2566) (width 0.5) (layer B.Cu) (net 4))
 (segment (start 146.7 88.7966) (end 145.1001 88.7966) (width 0.5) (layer B.Cu) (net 5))
 (segment (start 144.21 88.949) (end 144.9477 88.949) (width 0.5) (layer B.Cu) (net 5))
 (segment (start 144.9477 88.949) (end 145.1001 88.7966) (width 0.5) (layer B.Cu) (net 5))
 (segment (start 146.7 91.3366) (end 145.1001 91.3366) (width 0.5) (layer B.Cu) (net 6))
 (segment (start 144.21 91.489) (end 144.9477 91.489) (width 0.5) (layer B.Cu) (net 6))
 (segment (start 144.9477 91.489) (end 145.1001 91.3366) (width 0.5) (layer B.Cu) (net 6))
 (segment (start 146.7 93.8766) (end 145.1001 93.8766) (width 0.5) (layer B.Cu) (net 7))
 (segment (start 144.21 94.029) (end 144.9477 94.029) (width 0.5) (layer B.Cu) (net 7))
 (segment (start 144.9477 94.029) (end 145.1001 93.8766) (width 0.5) (layer B.Cu) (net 7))
 (segment (start 146.7 96.4166) (end 145.1001 96.4166) (width 0.5) (layer B.Cu) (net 8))
 (segment (start 144.21 96.569) (end 144.9477 96.569) (width 0.5) (layer B.Cu) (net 8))
 (segment (start 144.9477 96.569) (end 145.1001 96.4166) (width 0.5) (layer B.Cu) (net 8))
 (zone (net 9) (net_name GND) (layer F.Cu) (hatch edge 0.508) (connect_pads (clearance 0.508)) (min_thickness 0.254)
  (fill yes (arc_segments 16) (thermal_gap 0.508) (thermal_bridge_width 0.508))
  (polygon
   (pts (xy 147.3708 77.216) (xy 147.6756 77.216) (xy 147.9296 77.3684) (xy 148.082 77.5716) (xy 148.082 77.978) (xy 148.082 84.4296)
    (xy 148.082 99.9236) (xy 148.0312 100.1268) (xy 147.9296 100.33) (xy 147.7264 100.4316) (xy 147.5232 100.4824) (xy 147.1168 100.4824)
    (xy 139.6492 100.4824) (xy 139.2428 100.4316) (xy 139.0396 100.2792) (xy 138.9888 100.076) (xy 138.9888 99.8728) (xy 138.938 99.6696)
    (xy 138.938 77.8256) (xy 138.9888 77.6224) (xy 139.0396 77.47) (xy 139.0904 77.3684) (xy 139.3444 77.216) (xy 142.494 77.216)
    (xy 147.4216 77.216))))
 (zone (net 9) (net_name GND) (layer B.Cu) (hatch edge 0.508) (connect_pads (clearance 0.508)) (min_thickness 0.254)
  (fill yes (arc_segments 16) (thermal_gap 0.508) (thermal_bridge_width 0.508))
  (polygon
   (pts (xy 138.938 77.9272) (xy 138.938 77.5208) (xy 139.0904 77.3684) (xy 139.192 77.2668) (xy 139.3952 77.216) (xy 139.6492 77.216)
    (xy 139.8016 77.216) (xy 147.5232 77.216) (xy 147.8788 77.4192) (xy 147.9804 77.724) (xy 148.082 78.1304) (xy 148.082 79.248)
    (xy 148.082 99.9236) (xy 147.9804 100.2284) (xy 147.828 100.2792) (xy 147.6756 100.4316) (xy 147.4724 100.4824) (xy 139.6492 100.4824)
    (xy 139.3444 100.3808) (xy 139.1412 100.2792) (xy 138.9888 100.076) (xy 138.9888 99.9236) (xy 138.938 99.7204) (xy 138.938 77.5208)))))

